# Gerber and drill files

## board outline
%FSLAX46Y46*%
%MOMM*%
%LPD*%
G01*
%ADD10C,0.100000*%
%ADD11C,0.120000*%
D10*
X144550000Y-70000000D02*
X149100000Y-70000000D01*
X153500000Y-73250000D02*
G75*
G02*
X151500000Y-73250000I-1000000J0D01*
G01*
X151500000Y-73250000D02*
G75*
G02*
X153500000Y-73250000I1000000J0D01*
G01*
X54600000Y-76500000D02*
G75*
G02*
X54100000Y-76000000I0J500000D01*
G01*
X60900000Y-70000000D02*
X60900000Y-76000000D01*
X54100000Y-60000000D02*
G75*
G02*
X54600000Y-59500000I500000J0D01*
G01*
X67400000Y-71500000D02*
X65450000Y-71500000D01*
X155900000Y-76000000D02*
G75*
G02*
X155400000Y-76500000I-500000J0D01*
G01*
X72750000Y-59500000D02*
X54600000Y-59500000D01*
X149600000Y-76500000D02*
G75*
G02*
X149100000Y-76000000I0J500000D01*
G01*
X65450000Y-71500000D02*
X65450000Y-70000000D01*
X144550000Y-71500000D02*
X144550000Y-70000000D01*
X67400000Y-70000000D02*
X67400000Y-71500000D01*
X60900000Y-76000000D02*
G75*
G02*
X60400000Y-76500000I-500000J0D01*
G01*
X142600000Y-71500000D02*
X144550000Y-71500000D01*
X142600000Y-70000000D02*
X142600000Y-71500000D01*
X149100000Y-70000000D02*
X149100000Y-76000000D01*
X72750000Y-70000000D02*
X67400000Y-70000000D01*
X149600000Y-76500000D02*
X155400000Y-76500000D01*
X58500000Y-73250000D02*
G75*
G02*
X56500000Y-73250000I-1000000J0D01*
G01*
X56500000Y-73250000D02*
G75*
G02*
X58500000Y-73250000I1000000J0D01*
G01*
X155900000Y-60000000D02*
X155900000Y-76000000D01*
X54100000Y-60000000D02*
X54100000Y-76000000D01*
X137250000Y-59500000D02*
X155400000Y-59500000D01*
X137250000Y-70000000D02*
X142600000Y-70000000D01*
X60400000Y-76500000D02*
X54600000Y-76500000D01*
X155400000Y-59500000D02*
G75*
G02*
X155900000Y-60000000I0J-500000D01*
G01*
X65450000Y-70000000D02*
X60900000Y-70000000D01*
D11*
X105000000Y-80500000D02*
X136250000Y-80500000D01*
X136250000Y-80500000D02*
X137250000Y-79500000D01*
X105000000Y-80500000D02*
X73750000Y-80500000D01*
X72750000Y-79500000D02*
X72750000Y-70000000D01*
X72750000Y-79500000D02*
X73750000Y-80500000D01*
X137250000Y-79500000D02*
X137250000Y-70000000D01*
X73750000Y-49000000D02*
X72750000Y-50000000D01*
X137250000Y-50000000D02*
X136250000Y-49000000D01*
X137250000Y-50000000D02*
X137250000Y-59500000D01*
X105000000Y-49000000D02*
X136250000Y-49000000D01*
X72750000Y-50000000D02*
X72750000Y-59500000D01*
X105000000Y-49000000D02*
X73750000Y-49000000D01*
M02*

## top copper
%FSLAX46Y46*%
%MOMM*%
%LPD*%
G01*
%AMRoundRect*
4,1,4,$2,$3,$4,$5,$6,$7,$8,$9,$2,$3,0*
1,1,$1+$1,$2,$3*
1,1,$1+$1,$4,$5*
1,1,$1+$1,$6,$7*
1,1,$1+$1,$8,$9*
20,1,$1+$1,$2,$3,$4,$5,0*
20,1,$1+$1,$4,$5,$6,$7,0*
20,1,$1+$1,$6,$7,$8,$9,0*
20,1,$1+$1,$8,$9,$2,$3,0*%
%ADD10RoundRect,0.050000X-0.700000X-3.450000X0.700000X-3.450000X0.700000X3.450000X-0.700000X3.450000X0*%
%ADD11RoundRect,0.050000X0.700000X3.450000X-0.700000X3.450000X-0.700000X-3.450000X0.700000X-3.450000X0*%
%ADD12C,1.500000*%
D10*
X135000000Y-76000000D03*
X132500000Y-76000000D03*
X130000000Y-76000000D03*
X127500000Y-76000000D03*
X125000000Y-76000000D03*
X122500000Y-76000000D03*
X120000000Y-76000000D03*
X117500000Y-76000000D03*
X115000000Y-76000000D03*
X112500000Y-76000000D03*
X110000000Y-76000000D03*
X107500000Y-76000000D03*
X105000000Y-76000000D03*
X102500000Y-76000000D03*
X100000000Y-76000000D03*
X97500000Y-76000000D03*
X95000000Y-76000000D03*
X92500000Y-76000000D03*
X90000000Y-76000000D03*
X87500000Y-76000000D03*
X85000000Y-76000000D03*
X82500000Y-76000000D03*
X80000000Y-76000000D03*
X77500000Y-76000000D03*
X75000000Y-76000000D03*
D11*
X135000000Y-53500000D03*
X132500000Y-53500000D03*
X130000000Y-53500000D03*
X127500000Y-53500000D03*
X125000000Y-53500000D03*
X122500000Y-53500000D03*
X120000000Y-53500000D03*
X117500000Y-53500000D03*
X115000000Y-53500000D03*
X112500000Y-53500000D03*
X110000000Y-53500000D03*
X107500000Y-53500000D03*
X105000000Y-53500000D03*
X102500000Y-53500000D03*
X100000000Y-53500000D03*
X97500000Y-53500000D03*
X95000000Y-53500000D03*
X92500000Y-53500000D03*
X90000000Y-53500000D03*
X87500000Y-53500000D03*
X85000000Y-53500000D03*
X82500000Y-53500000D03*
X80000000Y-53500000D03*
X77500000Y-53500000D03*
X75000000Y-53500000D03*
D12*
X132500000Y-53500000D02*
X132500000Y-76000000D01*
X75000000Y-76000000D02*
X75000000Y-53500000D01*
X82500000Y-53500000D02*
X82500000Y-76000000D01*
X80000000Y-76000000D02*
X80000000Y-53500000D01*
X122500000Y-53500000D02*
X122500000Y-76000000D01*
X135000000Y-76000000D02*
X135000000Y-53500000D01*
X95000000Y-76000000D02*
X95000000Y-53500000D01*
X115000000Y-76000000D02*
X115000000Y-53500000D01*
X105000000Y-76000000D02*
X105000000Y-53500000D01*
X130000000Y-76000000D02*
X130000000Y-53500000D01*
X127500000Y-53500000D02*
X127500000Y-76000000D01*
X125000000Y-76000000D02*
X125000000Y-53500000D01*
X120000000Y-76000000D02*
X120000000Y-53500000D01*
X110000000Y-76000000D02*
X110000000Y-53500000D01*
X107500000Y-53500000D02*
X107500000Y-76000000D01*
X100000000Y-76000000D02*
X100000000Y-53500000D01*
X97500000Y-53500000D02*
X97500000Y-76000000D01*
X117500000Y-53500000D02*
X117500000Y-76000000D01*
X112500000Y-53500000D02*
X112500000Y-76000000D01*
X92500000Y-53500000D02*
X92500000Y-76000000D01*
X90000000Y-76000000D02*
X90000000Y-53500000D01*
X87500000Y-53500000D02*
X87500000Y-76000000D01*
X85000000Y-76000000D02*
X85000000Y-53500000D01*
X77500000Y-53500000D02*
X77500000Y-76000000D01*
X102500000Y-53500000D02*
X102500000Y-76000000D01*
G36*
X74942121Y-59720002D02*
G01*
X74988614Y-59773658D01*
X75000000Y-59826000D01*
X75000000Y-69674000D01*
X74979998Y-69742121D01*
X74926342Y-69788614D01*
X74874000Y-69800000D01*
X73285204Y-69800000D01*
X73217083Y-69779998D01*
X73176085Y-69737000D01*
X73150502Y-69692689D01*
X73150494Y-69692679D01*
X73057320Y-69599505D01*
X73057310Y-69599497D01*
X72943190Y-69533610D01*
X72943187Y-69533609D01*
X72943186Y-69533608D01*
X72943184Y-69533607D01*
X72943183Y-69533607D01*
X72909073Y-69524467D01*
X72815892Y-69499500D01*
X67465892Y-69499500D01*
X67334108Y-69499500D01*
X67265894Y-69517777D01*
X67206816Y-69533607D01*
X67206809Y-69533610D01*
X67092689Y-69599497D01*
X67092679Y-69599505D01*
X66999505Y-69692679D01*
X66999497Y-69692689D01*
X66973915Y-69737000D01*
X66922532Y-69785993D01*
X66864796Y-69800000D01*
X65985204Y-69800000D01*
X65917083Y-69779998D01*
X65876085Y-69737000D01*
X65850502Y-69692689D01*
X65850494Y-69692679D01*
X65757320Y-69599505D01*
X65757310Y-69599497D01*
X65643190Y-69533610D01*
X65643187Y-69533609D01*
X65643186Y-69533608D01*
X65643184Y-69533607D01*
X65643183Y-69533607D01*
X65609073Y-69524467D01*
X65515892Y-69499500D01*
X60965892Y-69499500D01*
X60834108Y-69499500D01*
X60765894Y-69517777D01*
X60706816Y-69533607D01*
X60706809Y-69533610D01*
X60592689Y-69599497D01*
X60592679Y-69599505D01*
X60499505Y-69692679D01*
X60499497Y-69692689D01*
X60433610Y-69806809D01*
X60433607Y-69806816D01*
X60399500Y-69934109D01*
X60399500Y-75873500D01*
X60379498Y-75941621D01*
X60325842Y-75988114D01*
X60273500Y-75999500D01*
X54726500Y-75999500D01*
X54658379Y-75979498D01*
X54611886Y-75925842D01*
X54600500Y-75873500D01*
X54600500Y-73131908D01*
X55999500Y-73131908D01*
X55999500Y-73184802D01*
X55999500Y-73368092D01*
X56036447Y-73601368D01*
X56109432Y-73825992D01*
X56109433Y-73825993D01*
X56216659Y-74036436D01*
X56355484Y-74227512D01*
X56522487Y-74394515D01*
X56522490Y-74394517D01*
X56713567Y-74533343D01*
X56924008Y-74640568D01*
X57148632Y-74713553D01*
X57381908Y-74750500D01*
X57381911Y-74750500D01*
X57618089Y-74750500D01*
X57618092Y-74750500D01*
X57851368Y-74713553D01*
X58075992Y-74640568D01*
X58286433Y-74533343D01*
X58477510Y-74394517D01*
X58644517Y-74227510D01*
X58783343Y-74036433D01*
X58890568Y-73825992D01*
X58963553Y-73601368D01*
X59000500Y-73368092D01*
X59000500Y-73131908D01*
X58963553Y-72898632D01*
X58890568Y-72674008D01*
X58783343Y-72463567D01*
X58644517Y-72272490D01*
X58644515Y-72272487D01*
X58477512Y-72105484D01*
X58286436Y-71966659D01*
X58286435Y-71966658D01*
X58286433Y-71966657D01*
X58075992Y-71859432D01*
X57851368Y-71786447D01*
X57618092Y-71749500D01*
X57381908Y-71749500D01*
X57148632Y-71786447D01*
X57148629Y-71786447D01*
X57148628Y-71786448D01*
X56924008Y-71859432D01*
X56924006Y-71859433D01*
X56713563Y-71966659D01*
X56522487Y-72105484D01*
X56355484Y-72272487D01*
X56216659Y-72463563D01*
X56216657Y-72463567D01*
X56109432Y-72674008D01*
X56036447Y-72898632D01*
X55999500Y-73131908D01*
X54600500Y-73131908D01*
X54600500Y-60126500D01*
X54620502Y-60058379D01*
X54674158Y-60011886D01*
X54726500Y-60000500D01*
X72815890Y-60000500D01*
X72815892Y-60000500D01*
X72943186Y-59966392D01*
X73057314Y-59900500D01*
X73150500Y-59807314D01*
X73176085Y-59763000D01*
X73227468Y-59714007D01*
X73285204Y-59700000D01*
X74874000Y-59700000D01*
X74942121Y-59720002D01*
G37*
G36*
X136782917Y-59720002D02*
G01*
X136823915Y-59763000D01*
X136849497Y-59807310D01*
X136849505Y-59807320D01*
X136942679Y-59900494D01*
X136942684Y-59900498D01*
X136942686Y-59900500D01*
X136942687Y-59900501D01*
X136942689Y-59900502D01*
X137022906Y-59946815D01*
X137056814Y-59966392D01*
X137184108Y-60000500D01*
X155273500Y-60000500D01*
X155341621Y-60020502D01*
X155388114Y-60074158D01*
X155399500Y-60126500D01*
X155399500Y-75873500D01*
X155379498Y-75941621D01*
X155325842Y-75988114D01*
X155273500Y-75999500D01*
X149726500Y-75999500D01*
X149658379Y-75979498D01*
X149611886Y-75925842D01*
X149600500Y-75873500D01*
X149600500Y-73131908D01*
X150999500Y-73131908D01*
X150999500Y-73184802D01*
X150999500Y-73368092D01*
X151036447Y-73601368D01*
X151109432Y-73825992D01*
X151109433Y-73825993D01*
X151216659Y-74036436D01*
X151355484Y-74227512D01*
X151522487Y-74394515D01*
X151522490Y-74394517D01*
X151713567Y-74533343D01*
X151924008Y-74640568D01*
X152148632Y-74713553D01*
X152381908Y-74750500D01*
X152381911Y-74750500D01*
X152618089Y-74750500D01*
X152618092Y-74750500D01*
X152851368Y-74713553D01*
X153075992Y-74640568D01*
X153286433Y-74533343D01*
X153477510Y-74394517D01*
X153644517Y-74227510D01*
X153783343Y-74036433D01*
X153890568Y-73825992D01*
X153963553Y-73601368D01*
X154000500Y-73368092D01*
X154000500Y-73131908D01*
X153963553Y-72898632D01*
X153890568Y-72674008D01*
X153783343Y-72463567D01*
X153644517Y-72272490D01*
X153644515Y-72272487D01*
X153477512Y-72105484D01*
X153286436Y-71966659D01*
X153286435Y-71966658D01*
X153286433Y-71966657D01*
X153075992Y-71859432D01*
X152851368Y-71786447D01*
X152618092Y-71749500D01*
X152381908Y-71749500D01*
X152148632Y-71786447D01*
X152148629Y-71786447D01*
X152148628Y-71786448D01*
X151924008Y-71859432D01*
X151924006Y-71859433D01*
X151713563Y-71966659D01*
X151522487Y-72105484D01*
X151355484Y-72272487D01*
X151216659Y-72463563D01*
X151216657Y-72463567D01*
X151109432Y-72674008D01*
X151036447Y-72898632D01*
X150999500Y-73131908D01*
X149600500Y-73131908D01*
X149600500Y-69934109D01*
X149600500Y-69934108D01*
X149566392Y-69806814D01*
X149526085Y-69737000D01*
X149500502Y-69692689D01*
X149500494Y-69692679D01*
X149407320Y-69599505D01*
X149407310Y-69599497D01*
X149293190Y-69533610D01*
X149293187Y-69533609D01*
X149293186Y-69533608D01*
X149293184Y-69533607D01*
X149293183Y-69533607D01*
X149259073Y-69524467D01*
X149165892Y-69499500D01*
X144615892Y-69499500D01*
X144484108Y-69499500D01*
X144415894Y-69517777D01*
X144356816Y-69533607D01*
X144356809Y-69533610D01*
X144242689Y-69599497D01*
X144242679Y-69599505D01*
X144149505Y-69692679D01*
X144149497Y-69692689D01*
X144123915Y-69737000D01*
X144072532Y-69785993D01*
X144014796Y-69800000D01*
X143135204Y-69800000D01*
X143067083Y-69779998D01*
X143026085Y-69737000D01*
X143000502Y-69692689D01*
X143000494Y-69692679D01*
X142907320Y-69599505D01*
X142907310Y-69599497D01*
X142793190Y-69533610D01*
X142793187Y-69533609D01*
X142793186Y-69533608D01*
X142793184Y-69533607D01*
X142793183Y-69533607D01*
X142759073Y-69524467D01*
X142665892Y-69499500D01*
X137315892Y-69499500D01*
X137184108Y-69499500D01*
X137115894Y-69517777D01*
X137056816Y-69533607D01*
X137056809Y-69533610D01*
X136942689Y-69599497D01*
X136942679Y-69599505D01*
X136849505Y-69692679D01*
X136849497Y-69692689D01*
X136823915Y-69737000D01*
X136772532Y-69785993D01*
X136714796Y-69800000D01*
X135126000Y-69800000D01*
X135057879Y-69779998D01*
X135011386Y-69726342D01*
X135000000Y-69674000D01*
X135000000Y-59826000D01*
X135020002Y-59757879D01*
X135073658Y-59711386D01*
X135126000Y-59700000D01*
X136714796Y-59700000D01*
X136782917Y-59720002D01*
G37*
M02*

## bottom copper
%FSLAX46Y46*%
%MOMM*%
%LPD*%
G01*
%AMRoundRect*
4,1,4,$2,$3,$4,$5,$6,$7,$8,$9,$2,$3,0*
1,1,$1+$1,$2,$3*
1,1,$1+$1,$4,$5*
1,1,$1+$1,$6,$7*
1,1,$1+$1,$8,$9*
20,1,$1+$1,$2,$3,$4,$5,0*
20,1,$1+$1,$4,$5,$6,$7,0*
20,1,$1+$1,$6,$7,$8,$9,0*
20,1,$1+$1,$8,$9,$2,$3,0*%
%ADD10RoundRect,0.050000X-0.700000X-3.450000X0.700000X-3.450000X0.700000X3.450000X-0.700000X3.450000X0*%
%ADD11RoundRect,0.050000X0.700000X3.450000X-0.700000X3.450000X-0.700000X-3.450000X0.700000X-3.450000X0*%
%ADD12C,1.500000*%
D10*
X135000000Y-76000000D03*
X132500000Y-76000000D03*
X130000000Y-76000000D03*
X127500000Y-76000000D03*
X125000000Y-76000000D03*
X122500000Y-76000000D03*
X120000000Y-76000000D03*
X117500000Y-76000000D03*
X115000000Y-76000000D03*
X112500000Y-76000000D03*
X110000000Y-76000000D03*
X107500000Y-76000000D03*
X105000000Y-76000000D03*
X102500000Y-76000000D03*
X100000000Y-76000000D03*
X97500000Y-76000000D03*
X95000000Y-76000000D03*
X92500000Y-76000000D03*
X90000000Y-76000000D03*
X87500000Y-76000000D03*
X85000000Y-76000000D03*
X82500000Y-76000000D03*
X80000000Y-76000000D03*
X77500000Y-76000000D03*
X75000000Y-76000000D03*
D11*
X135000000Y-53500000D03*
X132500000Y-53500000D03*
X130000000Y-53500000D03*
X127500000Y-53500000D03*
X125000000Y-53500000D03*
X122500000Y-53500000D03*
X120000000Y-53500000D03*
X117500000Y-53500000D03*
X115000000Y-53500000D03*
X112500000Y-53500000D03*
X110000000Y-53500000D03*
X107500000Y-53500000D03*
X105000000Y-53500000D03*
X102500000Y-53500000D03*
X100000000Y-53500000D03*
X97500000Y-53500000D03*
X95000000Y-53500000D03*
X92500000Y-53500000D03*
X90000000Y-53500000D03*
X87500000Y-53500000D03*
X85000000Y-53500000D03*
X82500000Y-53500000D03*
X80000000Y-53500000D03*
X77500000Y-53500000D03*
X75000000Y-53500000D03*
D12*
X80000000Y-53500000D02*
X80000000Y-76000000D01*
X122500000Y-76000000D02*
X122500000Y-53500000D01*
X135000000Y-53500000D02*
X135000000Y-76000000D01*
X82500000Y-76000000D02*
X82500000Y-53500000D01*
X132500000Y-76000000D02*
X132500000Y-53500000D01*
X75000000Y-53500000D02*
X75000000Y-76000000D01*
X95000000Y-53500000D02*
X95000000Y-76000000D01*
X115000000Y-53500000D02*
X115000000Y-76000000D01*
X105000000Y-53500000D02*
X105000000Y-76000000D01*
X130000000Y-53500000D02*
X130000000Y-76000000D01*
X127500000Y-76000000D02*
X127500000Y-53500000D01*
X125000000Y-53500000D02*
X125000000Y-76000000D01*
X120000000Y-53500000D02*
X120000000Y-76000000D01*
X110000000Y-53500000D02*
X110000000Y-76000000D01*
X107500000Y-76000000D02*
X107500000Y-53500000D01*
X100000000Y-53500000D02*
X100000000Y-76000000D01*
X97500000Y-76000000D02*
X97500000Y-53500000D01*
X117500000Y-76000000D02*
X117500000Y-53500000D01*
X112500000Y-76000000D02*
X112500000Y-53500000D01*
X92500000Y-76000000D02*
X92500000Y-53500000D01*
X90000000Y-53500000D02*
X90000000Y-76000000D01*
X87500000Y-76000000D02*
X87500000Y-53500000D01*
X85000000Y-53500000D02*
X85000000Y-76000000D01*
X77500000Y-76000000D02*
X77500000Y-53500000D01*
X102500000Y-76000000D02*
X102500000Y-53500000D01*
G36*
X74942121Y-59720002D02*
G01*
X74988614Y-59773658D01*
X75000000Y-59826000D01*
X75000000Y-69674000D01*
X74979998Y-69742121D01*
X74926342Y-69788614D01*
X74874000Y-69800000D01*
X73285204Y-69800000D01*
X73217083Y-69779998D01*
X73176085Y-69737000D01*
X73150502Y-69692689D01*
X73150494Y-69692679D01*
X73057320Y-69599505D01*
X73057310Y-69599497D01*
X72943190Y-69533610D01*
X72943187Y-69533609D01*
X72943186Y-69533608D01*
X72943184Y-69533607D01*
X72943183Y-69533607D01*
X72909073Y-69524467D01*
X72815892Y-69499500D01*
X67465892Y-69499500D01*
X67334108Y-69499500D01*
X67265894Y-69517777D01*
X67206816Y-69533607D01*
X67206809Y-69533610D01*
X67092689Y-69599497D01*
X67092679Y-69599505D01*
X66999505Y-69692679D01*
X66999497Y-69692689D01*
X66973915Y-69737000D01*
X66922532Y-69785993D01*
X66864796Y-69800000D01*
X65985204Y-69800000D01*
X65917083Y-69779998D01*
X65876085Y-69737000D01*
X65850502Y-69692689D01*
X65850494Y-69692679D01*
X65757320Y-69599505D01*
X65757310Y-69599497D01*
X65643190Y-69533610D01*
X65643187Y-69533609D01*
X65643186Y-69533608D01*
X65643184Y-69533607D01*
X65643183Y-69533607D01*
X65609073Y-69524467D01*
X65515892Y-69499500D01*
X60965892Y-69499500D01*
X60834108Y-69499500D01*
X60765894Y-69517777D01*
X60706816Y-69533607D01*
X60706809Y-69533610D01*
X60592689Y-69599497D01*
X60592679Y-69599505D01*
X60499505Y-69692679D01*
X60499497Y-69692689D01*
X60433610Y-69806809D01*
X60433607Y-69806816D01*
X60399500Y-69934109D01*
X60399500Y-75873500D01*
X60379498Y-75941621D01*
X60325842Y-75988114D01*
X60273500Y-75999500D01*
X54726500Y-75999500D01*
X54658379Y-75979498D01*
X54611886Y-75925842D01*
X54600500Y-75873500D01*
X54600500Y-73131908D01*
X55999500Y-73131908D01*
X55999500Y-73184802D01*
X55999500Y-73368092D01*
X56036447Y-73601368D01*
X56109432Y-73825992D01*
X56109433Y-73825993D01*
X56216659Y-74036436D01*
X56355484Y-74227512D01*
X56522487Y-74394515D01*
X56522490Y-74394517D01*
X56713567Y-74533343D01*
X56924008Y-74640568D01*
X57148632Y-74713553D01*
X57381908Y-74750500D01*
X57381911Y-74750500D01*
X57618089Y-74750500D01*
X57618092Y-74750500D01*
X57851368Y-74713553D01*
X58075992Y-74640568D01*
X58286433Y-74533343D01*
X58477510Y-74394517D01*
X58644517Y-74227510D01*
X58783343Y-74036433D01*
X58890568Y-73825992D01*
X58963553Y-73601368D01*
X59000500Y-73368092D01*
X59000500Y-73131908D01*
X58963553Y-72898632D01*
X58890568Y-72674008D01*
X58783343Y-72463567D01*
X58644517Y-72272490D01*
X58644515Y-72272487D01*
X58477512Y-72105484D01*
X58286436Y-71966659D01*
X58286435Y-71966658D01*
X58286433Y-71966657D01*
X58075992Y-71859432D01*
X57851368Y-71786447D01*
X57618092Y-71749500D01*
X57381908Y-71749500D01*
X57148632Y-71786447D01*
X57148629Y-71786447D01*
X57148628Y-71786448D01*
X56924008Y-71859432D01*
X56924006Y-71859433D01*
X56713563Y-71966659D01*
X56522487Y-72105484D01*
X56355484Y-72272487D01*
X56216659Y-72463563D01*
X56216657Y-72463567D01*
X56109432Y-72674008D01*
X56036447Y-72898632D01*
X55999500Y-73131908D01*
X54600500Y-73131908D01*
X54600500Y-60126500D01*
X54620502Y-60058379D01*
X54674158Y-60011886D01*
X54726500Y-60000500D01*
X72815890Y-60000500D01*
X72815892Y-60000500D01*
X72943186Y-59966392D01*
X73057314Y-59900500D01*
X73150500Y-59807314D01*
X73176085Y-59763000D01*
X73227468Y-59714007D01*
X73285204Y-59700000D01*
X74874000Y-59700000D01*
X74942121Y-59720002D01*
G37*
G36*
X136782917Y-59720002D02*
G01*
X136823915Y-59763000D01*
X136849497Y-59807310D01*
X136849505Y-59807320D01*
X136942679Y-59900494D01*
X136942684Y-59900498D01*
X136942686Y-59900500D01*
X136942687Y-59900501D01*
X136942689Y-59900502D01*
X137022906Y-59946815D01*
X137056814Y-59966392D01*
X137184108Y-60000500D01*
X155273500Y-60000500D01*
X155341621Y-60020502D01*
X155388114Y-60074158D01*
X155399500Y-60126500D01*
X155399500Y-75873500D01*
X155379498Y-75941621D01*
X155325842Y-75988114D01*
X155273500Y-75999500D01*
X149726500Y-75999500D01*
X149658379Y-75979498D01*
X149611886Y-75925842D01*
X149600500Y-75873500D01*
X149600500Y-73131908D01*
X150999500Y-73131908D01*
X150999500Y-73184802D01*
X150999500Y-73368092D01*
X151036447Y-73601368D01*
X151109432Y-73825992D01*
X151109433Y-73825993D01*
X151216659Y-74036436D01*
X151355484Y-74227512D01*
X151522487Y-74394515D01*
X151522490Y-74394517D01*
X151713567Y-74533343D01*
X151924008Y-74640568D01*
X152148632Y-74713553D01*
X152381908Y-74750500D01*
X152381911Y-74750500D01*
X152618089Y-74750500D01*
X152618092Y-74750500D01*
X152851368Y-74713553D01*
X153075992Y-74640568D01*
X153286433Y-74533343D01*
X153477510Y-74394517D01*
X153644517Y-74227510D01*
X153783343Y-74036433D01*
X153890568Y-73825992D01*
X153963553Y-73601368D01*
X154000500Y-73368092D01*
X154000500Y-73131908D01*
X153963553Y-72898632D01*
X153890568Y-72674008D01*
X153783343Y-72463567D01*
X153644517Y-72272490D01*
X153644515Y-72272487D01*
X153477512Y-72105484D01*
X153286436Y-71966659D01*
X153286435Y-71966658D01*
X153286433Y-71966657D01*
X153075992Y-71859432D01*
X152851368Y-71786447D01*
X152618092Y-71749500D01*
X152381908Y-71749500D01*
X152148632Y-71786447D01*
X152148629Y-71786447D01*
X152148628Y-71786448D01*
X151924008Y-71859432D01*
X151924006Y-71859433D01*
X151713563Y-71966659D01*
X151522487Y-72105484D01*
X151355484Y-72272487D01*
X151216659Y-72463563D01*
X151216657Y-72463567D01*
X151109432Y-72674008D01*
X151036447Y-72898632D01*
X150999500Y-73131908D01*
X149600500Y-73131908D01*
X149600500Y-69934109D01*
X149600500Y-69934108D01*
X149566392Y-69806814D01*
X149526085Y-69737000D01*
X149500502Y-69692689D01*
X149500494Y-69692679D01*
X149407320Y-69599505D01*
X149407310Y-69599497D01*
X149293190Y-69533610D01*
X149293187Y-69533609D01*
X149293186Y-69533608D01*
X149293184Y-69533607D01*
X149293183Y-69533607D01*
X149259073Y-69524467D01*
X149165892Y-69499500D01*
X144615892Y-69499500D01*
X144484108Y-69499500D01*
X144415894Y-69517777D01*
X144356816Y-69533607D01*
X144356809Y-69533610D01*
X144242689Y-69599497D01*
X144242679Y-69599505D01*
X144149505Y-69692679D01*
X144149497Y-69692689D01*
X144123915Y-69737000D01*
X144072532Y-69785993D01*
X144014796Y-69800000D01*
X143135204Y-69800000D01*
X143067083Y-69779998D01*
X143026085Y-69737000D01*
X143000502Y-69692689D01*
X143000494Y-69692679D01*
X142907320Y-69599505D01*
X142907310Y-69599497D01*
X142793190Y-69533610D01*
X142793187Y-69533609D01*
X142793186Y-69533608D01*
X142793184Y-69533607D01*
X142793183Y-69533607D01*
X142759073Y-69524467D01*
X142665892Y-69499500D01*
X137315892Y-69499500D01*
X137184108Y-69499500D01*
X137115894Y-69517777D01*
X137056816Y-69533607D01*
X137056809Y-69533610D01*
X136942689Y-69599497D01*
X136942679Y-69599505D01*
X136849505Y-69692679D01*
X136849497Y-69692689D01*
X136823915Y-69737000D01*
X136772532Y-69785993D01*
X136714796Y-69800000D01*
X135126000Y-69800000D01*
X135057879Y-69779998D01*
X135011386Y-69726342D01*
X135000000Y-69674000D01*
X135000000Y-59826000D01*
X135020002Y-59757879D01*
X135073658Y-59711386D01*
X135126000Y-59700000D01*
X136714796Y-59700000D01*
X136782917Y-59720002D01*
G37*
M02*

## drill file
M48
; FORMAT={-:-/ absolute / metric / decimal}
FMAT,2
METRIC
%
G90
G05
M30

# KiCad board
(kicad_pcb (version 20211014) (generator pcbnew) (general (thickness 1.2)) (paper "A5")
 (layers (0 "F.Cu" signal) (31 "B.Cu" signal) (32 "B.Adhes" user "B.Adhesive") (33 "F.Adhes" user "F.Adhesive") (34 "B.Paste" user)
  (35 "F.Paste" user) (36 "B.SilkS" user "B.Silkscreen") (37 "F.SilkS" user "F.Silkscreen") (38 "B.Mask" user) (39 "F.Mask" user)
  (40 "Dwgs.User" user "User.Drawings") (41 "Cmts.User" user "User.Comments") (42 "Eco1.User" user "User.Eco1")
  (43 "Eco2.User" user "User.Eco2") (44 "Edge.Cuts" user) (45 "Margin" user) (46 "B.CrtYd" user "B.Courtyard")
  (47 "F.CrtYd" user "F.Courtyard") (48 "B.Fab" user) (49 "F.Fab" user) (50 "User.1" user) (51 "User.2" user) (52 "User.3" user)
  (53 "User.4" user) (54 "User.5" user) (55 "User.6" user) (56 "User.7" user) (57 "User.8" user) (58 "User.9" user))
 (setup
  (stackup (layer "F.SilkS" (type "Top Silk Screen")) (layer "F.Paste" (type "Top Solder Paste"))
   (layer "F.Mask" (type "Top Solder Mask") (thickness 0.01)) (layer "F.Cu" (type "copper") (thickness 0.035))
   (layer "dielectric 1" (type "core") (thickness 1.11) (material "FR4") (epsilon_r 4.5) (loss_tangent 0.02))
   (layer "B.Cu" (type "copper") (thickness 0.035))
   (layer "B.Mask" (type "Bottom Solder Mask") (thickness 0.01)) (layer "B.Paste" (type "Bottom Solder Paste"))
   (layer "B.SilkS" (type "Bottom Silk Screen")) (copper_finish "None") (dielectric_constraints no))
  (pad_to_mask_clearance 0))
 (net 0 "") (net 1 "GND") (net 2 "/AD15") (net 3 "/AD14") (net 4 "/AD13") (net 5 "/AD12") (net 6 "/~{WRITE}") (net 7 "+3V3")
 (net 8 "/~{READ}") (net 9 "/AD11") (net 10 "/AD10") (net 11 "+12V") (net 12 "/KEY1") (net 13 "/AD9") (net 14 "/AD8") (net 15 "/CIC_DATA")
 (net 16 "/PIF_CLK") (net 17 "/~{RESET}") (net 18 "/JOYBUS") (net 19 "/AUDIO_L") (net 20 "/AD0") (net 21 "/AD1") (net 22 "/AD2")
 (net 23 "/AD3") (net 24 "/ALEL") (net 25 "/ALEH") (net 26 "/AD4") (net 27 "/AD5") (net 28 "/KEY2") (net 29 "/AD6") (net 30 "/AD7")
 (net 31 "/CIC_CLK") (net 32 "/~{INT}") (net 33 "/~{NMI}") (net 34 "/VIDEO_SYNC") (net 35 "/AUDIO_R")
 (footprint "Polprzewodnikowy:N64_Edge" (layer "F.Cu") (at 105 70)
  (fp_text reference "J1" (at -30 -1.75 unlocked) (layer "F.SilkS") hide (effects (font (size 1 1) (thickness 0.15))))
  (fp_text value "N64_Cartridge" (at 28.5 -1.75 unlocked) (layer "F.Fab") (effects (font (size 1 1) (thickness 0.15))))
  (fp_line (start 0 10.5) (end 31.25 10.5) (layer "Edge.Cuts") (width 0.12))
  (fp_line (start 31.25 10.5) (end 32.25 9.5) (layer "Edge.Cuts") (width 0.12))
  (fp_line (start 0 10.5) (end -31.25 10.5) (layer "Edge.Cuts") (width 0.12))
  (fp_line (start -32.25 9.5) (end -32.25 0) (layer "Edge.Cuts") (width 0.12))
  (fp_line (start -32.25 9.5) (end -31.25 10.5) (layer "Edge.Cuts") (width 0.12))
  (fp_line (start 32.25 9.5) (end 32.25 0) (layer "Edge.Cuts") (width 0.12))
  (pad "1" connect roundrect (at 30 6) (size 1.5 7) (layers "B.Cu") (roundrect_rratio 0.03333333333) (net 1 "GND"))
  (pad "2" connect roundrect (at 27.5 6) (size 1.5 7) (layers "B.Cu") (roundrect_rratio 0.03333333333) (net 1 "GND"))
  (pad "3" connect roundrect (at 25 6) (size 1.5 7) (layers "B.Cu") (roundrect_rratio 0.03333333333) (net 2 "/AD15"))
  (pad "4" connect roundrect (at 22.5 6) (size 1.5 7) (layers "B.Cu") (roundrect_rratio 0.03333333333) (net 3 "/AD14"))
  (pad "5" connect roundrect (at 20 6) (size 1.5 7) (layers "B.Cu") (roundrect_rratio 0.03333333333) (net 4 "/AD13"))
  (pad "6" connect roundrect (at 17.5 6) (size 1.5 7) (layers "B.Cu") (roundrect_rratio 0.03333333333) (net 1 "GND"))
  (pad "7" connect roundrect (at 15 6) (size 1.5 7) (layers "B.Cu") (roundrect_rratio 0.03333333333) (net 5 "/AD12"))
  (pad "8" connect roundrect (at 12.5 6) (size 1.5 7) (layers "B.Cu") (roundrect_rratio 0.03333333333) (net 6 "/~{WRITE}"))
  (pad "9" connect roundrect (at 10 6) (size 1.5 7) (layers "B.Cu") (roundrect_rratio 0.03333333333) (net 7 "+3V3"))
  (pad "10" connect roundrect (at 7.5 6) (size 1.5 7) (layers "B.Cu") (roundrect_rratio 0.03333333333) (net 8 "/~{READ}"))
  (pad "11" connect roundrect (at 5 6) (size 1.5 7) (layers "B.Cu") (roundrect_rratio 0.03333333333) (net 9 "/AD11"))
  (pad "12" connect roundrect (at 2.5 6) (size 1.5 7) (layers "B.Cu") (roundrect_rratio 0.03333333333) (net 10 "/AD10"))
  (pad "13" connect roundrect (at 0 6) (size 1.5 7) (layers "B.Cu") (roundrect_rratio 0.03333333333) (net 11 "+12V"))
  (pad "14" connect roundrect (at -2.5 6) (size 1.5 7) (layers "B.Cu") (roundrect_rratio 0.03333333333) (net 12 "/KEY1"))
  (pad "15" connect roundrect (at -5 6) (size 1.5 7) (layers "B.Cu") (roundrect_rratio 0.03333333333) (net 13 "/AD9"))
  (pad "16" connect roundrect (at -7.5 6) (size 1.5 7) (layers "B.Cu") (roundrect_rratio 0.03333333333) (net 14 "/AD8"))
  (pad "17" connect roundrect (at -10 6) (size 1.5 7) (layers "B.Cu") (roundrect_rratio 0.03333333333) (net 7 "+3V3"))
  (pad "18" connect roundrect (at -12.5 6) (size 1.5 7) (layers "B.Cu") (roundrect_rratio 0.03333333333) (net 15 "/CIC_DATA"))
  (pad "19" connect roundrect (at -15 6) (size 1.5 7) (layers "B.Cu") (roundrect_rratio 0.03333333333) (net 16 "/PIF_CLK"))
  (pad "20" connect roundrect (at -17.5 6) (size 1.5 7) (layers "B.Cu") (roundrect_rratio 0.03333333333) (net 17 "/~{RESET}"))
  (pad "21" connect roundrect (at -20 6) (size 1.5 7) (layers "B.Cu") (roundrect_rratio 0.03333333333) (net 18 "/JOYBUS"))
  (pad "22" connect roundrect (at -22.5 6) (size 1.5 7) (layers "B.Cu") (roundrect_rratio 0.03333333333) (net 1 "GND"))
  (pad "23" connect roundrect (at -25 6) (size 1.5 7) (layers "B.Cu") (roundrect_rratio 0.03333333333) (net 1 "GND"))
  (pad "24" connect roundrect (at -27.5 6) (size 1.5 7) (layers "B.Cu") (roundrect_rratio 0.03333333333) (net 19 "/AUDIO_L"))
  (pad "25" connect roundrect (at -30 6) (size 1.5 7) (layers "B.Cu") (roundrect_rratio 0.03333333333) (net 1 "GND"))
  (pad "26" connect roundrect (at 30 6) (size 1.5 7) (layers "F.Cu") (roundrect_rratio 0.03333333333) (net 1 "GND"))
  (pad "27" connect roundrect (at 27.5 6) (size 1.5 7) (layers "F.Cu") (roundrect_rratio 0.03333333333) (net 1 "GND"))
  (pad "28" connect roundrect (at 25 6) (size 1.5 7) (layers "F.Cu") (roundrect_rratio 0.03333333333) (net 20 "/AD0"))
  (pad "29" connect roundrect (at 22.5 6) (size 1.5 7) (layers "F.Cu") (roundrect_rratio 0.03333333333) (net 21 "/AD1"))
  (pad "30" connect roundrect (at 20 6) (size 1.5 7) (layers "F.Cu") (roundrect_rratio 0.03333333333) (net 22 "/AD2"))
  (pad "31" connect roundrect (at 17.5 6) (size 1.5 7) (layers "F.Cu") (roundrect_rratio 0.03333333333) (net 1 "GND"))
  (pad "32" connect roundrect (at 15 6) (size 1.5 7) (layers "F.Cu") (roundrect_rratio 0.03333333333) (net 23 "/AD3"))
  (pad "33" connect roundrect (at 12.5 6) (size 1.5 7) (layers "F.Cu") (roundrect_rratio 0.03333333333) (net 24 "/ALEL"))
  (pad "34" connect roundrect (at 10 6) (size 1.5 7) (layers "F.Cu") (roundrect_rratio 0.03333333333) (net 7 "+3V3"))
  (pad "35" connect roundrect (at 7.5 6) (size 1.5 7) (layers "F.Cu") (roundrect_rratio 0.03333333333) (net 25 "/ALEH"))
  (pad "36" connect roundrect (at 5 6) (size 1.5 7) (layers "F.Cu") (roundrect_rratio 0.03333333333) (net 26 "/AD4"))
  (pad "37" connect roundrect (at 2.5 6) (size 1.5 7) (layers "F.Cu") (roundrect_rratio 0.03333333333) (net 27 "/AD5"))
  (pad "38" connect roundrect (at 0 6) (size 1.5 7) (layers "F.Cu") (roundrect_rratio 0.03333333333) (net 11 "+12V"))
  (pad "39" connect roundrect (at -2.5 6) (size 1.5 7) (layers "F.Cu") (roundrect_rratio 0.03333333333) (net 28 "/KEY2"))
  (pad "40" connect roundrect (at -5 6) (size 1.5 7) (layers "F.Cu") (roundrect_rratio 0.03333333333) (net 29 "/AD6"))
  (pad "41" connect roundrect (at -7.5 6) (size 1.5 7) (layers "F.Cu") (roundrect_rratio 0.03333333333) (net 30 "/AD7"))
  (pad "42" connect roundrect (at -10 6) (size 1.5 7) (layers "F.Cu") (roundrect_rratio 0.03333333333) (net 7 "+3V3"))
  (pad "43" connect roundrect (at -12.5 6) (size 1.5 7) (layers "F.Cu") (roundrect_rratio 0.03333333333) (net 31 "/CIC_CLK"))
  (pad "44" connect roundrect (at -15 6) (size 1.5 7) (layers "F.Cu") (roundrect_rratio 0.03333333333) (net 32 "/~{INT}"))
  (pad "45" connect roundrect (at -17.5 6) (size 1.5 7) (layers "F.Cu") (roundrect_rratio 0.03333333333) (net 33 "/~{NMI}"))
  (pad "46" connect roundrect (at -20 6) (size 1.5 7) (layers "F.Cu") (roundrect_rratio 0.03333333333) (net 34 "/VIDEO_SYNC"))
  (pad "47" connect roundrect (at -22.5 6) (size 1.5 7) (layers "F.Cu") (roundrect_rratio 0.03333333333) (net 1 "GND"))
  (pad "48" connect roundrect (at -25 6) (size 1.5 7) (layers "F.Cu") (roundrect_rratio 0.03333333333) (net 1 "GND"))
  (pad "49" connect roundrect (at -27.5 6) (size 1.5 7) (layers "F.Cu") (roundrect_rratio 0.03333333333) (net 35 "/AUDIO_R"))
  (pad "50" connect roundrect (at -30 6) (size 1.5 7) (layers "F.Cu") (roundrect_rratio 0.03333333333) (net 1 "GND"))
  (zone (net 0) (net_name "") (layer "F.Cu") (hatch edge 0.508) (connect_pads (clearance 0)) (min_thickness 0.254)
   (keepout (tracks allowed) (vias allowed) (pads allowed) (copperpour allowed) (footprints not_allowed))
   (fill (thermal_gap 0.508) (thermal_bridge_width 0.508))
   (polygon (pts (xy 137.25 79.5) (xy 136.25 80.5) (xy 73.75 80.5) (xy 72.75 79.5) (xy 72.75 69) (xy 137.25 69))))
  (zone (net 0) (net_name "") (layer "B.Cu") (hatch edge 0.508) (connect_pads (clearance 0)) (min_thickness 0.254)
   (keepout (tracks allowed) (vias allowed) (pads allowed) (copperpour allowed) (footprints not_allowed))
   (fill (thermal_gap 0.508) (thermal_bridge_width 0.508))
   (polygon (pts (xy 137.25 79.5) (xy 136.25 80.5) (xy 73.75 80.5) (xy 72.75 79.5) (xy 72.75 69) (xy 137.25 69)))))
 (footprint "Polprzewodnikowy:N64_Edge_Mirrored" (layer "F.Cu") (at 105 59.5 180)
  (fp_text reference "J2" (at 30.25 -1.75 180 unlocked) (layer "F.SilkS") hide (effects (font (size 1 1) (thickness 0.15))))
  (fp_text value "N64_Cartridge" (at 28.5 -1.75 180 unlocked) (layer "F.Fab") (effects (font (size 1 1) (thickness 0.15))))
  (fp_line (start 31.25 10.5) (end 32.25 9.5) (layer "Edge.Cuts") (width 0.12))
  (fp_line (start -32.25 9.5) (end -31.25 10.5) (layer "Edge.Cuts") (width 0.12))
  (fp_line (start -32.25 9.5) (end -32.25 0) (layer "Edge.Cuts") (width 0.12))
  (fp_line (start 0 10.5) (end -31.25 10.5) (layer "Edge.Cuts") (width 0.12))
  (fp_line (start 32.25 9.5) (end 32.25 0) (layer "Edge.Cuts") (width 0.12))
  (fp_line (start 0 10.5) (end 31.25 10.5) (layer "Edge.Cuts") (width 0.12))
  (pad "1" connect roundrect (at -30 6 180) (size 1.5 7) (layers "B.Cu") (roundrect_rratio 0.03333333333) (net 1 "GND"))
  (pad "2" connect roundrect (at -27.5 6 180) (size 1.5 7) (layers "B.Cu") (roundrect_rratio 0.03333333333) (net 1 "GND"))
  (pad "3" connect roundrect (at -25 6 180) (size 1.5 7) (layers "B.Cu") (roundrect_rratio 0.03333333333) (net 2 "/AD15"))
  (pad "4" connect roundrect (at -22.5 6 180) (size 1.5 7) (layers "B.Cu") (roundrect_rratio 0.03333333333) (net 3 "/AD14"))
  (pad "5" connect roundrect (at -20 6 180) (size 1.5 7) (layers "B.Cu") (roundrect_rratio 0.03333333333) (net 4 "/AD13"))
  (pad "6" connect roundrect (at -17.5 6 180) (size 1.5 7) (layers "B.Cu") (roundrect_rratio 0.03333333333) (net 1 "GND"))
  (pad "7" connect roundrect (at -15 6 180) (size 1.5 7) (layers "B.Cu") (roundrect_rratio 0.03333333333) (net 5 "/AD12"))
  (pad "8" connect roundrect (at -12.5 6 180) (size 1.5 7) (layers "B.Cu") (roundrect_rratio 0.03333333333) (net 6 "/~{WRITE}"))
  (pad "9" connect roundrect (at -10 6 180) (size 1.5 7) (layers "B.Cu") (roundrect_rratio 0.03333333333) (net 7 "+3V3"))
  (pad "10" connect roundrect (at -7.5 6 180) (size 1.5 7) (layers "B.Cu") (roundrect_rratio 0.03333333333) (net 8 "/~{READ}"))
  (pad "11" connect roundrect (at -5 6 180) (size 1.5 7) (layers "B.Cu") (roundrect_rratio 0.03333333333) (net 9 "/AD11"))
  (pad "12" connect roundrect (at -2.5 6 180) (size 1.5 7) (layers "B.Cu") (roundrect_rratio 0.03333333333) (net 10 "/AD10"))
  (pad "13" connect roundrect (at 0 6 180) (size 1.5 7) (layers "B.Cu") (roundrect_rratio 0.03333333333) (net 11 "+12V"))
  (pad "14" connect roundrect (at 2.5 6 180) (size 1.5 7) (layers "B.Cu") (roundrect_rratio 0.03333333333) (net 12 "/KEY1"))
  (pad "15" connect roundrect (at 5 6 180) (size 1.5 7) (layers "B.Cu") (roundrect_rratio 0.03333333333) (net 13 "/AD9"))
  (pad "16" connect roundrect (at 7.5 6 180) (size 1.5 7) (layers "B.Cu") (roundrect_rratio 0.03333333333) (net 14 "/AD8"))
  (pad "17" connect roundrect (at 10 6 180) (size 1.5 7) (layers "B.Cu") (roundrect_rratio 0.03333333333) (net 7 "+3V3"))
  (pad "18" connect roundrect (at 12.5 6 180) (size 1.5 7) (layers "B.Cu") (roundrect_rratio 0.03333333333) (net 15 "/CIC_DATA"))
  (pad "19" connect roundrect (at 15 6 180) (size 1.5 7) (layers "B.Cu") (roundrect_rratio 0.03333333333) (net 16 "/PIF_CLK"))
  (pad "20" connect roundrect (at 17.5 6 180) (size 1.5 7) (layers "B.Cu") (roundrect_rratio 0.03333333333) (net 17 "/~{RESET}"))
  (pad "21" connect roundrect (at 20 6 180) (size 1.5 7) (layers "B.Cu") (roundrect_rratio 0.03333333333) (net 18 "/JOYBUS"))
  (pad "22" connect roundrect (at 22.5 6 180) (size 1.5 7) (layers "B.Cu") (roundrect_rratio 0.03333333333) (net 1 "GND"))
  (pad "23" connect roundrect (at 25 6 180) (size 1.5 7) (layers "B.Cu") (roundrect_rratio 0.03333333333) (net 1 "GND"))
  (pad "24" connect roundrect (at 27.5 6 180) (size 1.5 7) (layers "B.Cu") (roundrect_rratio 0.03333333333) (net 19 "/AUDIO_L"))
  (pad "25" connect roundrect (at 30 6 180) (size 1.5 7) (layers "B.Cu") (roundrect_rratio 0.03333333333) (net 1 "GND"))
  (pad "26" connect roundrect (at -30 6 180) (size 1.5 7) (layers "F.Cu") (roundrect_rratio 0.03333333333) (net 1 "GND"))
  (pad "27" connect roundrect (at -27.5 6 180) (size 1.5 7) (layers "F.Cu") (roundrect_rratio 0.03333333333) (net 1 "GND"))
  (pad "28" connect roundrect (at -25 6 180) (size 1.5 7) (layers "F.Cu") (roundrect_rratio 0.03333333333) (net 20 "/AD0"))
  (pad "29" connect roundrect (at -22.5 6 180) (size 1.5 7) (layers "F.Cu") (roundrect_rratio 0.03333333333) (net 21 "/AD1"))
  (pad "30" connect roundrect (at -20 6 180) (size 1.5 7) (layers "F.Cu") (roundrect_rratio 0.03333333333) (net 22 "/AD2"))
  (pad "31" connect roundrect (at -17.5 6 180) (size 1.5 7) (layers "F.Cu") (roundrect_rratio 0.03333333333) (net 1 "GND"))
  (pad "32" connect roundrect (at -15 6 180) (size 1.5 7) (layers "F.Cu") (roundrect_rratio 0.03333333333) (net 23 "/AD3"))
  (pad "33" connect roundrect (at -12.5 6 180) (size 1.5 7) (layers "F.Cu") (roundrect_rratio 0.03333333333) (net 24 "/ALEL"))
  (pad "34" connect roundrect (at -10 6 180) (size 1.5 7) (layers "F.Cu") (roundrect_rratio 0.03333333333) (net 7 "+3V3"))
  (pad "35" connect roundrect (at -7.5 6 180) (size 1.5 7) (layers "F.Cu") (roundrect_rratio 0.03333333333) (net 25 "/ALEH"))
  (pad "36" connect roundrect (at -5 6 180) (size 1.5 7) (layers "F.Cu") (roundrect_rratio 0.03333333333) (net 26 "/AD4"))
  (pad "37" connect roundrect (at -2.5 6 180) (size 1.5 7) (layers "F.Cu") (roundrect_rratio 0.03333333333) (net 27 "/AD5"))
  (pad "38" connect roundrect (at 0 6 180) (size 1.5 7) (layers "F.Cu") (roundrect_rratio 0.03333333333) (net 11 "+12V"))
  (pad "39" connect roundrect (at 2.5 6 180) (size 1.5 7) (layers "F.Cu") (roundrect_rratio 0.03333333333) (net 28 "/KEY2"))
  (pad "40" connect roundrect (at 5 6 180) (size 1.5 7) (layers "F.Cu") (roundrect_rratio 0.03333333333) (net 29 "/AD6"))
  (pad "41" connect roundrect (at 7.5 6 180) (size 1.5 7) (layers "F.Cu") (roundrect_rratio 0.03333333333) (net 30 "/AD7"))
  (pad "42" connect roundrect (at 10 6 180) (size 1.5 7) (layers "F.Cu") (roundrect_rratio 0.03333333333) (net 7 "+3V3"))
  (pad "43" connect roundrect (at 12.5 6 180) (size 1.5 7) (layers "F.Cu") (roundrect_rratio 0.03333333333) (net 31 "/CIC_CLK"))
  (pad "44" connect roundrect (at 15 6 180) (size 1.5 7) (layers "F.Cu") (roundrect_rratio 0.03333333333) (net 32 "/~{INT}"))
  (pad "45" connect roundrect (at 17.5 6 180) (size 1.5 7) (layers "F.Cu") (roundrect_rratio 0.03333333333) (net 33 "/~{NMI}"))
  (pad "46" connect roundrect (at 20 6 180) (size 1.5 7) (layers "F.Cu") (roundrect_rratio 0.03333333333) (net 34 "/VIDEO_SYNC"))
  (pad "47" connect roundrect (at 22.5 6 180) (size 1.5 7) (layers "F.Cu") (roundrect_rratio 0.03333333333) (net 1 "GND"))
  (pad "48" connect roundrect (at 25 6 180) (size 1.5 7) (layers "F.Cu") (roundrect_rratio 0.03333333333) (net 1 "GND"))
  (pad "49" connect roundrect (at 27.5 6 180) (size 1.5 7) (layers "F.Cu") (roundrect_rratio 0.03333333333) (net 35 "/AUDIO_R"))
  (pad "50" connect roundrect (at 30 6 180) (size 1.5 7) (layers "F.Cu") (roundrect_rratio 0.03333333333) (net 1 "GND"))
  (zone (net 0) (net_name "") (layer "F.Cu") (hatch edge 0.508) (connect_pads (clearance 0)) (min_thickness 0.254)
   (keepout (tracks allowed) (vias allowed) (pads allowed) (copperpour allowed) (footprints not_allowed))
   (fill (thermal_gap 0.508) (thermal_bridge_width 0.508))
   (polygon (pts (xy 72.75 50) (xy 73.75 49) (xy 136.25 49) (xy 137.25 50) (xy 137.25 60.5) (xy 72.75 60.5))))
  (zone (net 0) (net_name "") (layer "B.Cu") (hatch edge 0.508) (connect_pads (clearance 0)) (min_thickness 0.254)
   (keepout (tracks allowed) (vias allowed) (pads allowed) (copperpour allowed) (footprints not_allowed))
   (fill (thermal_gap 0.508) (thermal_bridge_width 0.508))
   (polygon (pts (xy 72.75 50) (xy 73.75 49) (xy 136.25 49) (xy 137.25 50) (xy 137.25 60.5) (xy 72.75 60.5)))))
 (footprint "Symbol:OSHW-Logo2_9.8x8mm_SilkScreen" (layer "B.Cu") (at 66.5 64.75 180)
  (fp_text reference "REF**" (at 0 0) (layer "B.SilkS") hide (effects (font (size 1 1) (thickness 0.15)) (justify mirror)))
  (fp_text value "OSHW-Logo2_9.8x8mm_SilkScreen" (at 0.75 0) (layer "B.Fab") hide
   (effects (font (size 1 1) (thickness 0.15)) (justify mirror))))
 (gr_line (start 144.55 70) (end 149.1 70) (layer "Edge.Cuts") (width 0.1))
 (gr_circle (center 152.5 73.25) (end 153.5 73.25) (layer "Edge.Cuts") (width 0.1) (fill none))
 (gr_arc (start 54.6 76.5) (mid 54.246447 76.353553) (end 54.1 76) (layer "Edge.Cuts") (width 0.1))
 (gr_line (start 60.9 70) (end 60.9 76) (layer "Edge.Cuts") (width 0.1))
 (gr_arc (start 54.1 60) (mid 54.246447 59.646447) (end 54.6 59.5) (layer "Edge.Cuts") (width 0.1))
 (gr_line (start 67.4 71.5) (end 65.45 71.5) (layer "Edge.Cuts") (width 0.1))
 (gr_arc (start 155.9 76) (mid 155.753553 76.353553) (end 155.4 76.5) (layer "Edge.Cuts") (width 0.1))
 (gr_line (start 72.75 59.5) (end 54.6 59.5) (layer "Edge.Cuts") (width 0.1))
 (gr_arc (start 149.6 76.5) (mid 149.246447 76.353553) (end 149.1 76) (layer "Edge.Cuts") (width 0.1))
 (gr_line (start 65.45 71.5) (end 65.45 70) (layer "Edge.Cuts") (width 0.1))
 (gr_line (start 144.55 71.5) (end 144.55 70) (layer "Edge.Cuts") (width 0.1))
 (gr_line (start 67.4 70) (end 67.4 71.5) (layer "Edge.Cuts") (width 0.1))
 (gr_arc (start 60.9 76) (mid 60.753553 76.353553) (end 60.4 76.5) (layer "Edge.Cuts") (width 0.1))
 (gr_line (start 142.6 71.5) (end 144.55 71.5) (layer "Edge.Cuts") (width 0.1))
 (gr_line (start 142.6 70) (end 142.6 71.5) (layer "Edge.Cuts") (width 0.1))
 (gr_line (start 149.1 70) (end 149.1 76) (layer "Edge.Cuts") (width 0.1))
 (gr_line (start 72.75 70) (end 67.4 70) (layer "Edge.Cuts") (width 0.1))
 (gr_line (start 149.6 76.5) (end 155.4 76.5) (layer "Edge.Cuts") (width 0.1))
 (gr_circle (center 57.5 73.25) (end 58.5 73.25) (layer "Edge.Cuts") (width 0.1) (fill none))
 (gr_line (start 155.9 60) (end 155.9 76) (layer "Edge.Cuts") (width 0.1))
 (gr_line (start 54.1 60) (end 54.1 76) (layer "Edge.Cuts") (width 0.1))
 (gr_line (start 137.25 59.5) (end 155.4 59.5) (layer "Edge.Cuts") (width 0.1))
 (gr_line (start 137.25 70) (end 142.6 70) (layer "Edge.Cuts") (width 0.1))
 (gr_line (start 60.4 76.5) (end 54.6 76.5) (layer "Edge.Cuts") (width 0.1))
 (gr_arc (start 155.4 59.5) (mid 155.753553 59.646447) (end 155.9 60) (layer "Edge.Cuts") (width 0.1))
 (gr_line (start 65.45 70) (end 60.9 70) (layer "Edge.Cuts") (width 0.1))
 (segment (start 132.5 53.5) (end 132.5 76) (width 1.5) (layer "F.Cu") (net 1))
 (segment (start 75 76) (end 75 53.5) (width 1.5) (layer "F.Cu") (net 1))
 (segment (start 82.5 53.5) (end 82.5 76) (width 1.5) (layer "F.Cu") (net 1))
 (segment (start 80 76) (end 80 53.5) (width 1.5) (layer "F.Cu") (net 1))
 (segment (start 122.5 53.5) (end 122.5 76) (width 1.5) (layer "F.Cu") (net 1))
 (segment (start 135 76) (end 135 53.5) (width 1.5) (layer "F.Cu") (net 1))
 (segment (start 80 53.5) (end 80 76) (width 1.5) (layer "B.Cu") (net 1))
 (segment (start 122.5 76) (end 122.5 53.5) (width 1.5) (layer "B.Cu") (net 1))
 (segment (start 135 53.5) (end 135 76) (width 1.5) (layer "B.Cu") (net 1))
 (segment (start 82.5 76) (end 82.5 53.5) (width 1.5) (layer "B.Cu") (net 1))
 (segment (start 132.5 76) (end 132.5 53.5) (width 1.5) (layer "B.Cu") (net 1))
 (segment (start 75 53.5) (end 75 76) (width 1.5) (layer "B.Cu") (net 1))
 (segment (start 95 76) (end 95 53.5) (width 1.5) (layer "F.Cu") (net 7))
 (segment (start 115 76) (end 115 53.5) (width 1.5) (layer "F.Cu") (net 7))
 (segment (start 95 53.5) (end 95 76) (width 1.5) (layer "B.Cu") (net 7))
 (segment (start 115 53.5) (end 115 76) (width 1.5) (layer "B.Cu") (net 7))
 (segment (start 105 76) (end 105 53.5) (width 1.5) (layer "F.Cu") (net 11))
 (segment (start 105 53.5) (end 105 76) (width 1.5) (layer "B.Cu") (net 11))
 (segment (start 130 76) (end 130 53.5) (width 1.5) (layer "F.Cu") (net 20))
 (segment (start 127.5 53.5) (end 127.5 76) (width 1.5) (layer "F.Cu") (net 21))
 (segment (start 130 53.5) (end 130 76) (width 1.5) (layer "B.Cu") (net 2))
 (segment (start 127.5 76) (end 127.5 53.5) (width 1.5) (layer "B.Cu") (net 3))
 (segment (start 125 53.5) (end 125 76) (width 1.5) (layer "B.Cu") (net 4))
 (segment (start 120 53.5) (end 120 76) (width 1.5) (layer "B.Cu") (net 5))
 (segment (start 110 53.5) (end 110 76) (width 1.5) (layer "B.Cu") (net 9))
 (segment (start 107.5 76) (end 107.5 53.5) (width 1.5) (layer "B.Cu") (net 10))
 (segment (start 100 53.5) (end 100 76) (width 1.5) (layer "B.Cu") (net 13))
 (segment (start 97.5 76) (end 97.5 53.5) (width 1.5) (layer "B.Cu") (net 14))
 (segment (start 125 76) (end 125 53.5) (width 1.5) (layer "F.Cu") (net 22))
 (segment (start 120 76) (end 120 53.5) (width 1.5) (layer "F.Cu") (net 23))
 (segment (start 110 76) (end 110 53.5) (width 1.5) (layer "F.Cu") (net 26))
 (segment (start 107.5 53.5) (end 107.5 76) (width 1.5) (layer "F.Cu") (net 27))
 (segment (start 100 76) (end 100 53.5) (width 1.5) (layer "F.Cu") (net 29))
 (segment (start 97.5 53.5) (end 97.5 76) (width 1.5) (layer "F.Cu") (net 30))
 (segment (start 117.5 76) (end 117.5 53.5) (width 1.5) (layer "B.Cu") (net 6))
 (segment (start 112.5 76) (end 112.5 53.5) (width 1.5) (layer "B.Cu") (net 8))
 (segment (start 92.5 76) (end 92.5 53.5) (width 1.5) (layer "B.Cu") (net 15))
 (segment (start 90 53.5) (end 90 76) (width 1.5) (layer "B.Cu") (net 16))
 (segment (start 87.5 76) (end 87.5 53.5) (width 1.5) (layer "B.Cu") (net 17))
 (segment (start 85 53.5) (end 85 76) (width 1.5) (layer "B.Cu") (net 18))
 (segment (start 77.5 76) (end 77.5 53.5) (width 1.5) (layer "B.Cu") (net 19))
 (segment (start 117.5 53.5) (end 117.5 76) (width 1.5) (layer "F.Cu") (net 24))
 (segment (start 112.5 53.5) (end 112.5 76) (width 1.5) (layer "F.Cu") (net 25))
 (segment (start 92.5 53.5) (end 92.5 76) (width 1.5) (layer "F.Cu") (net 31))
 (segment (start 90 76) (end 90 53.5) (width 1.5) (layer "F.Cu") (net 32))
 (segment (start 87.5 53.5) (end 87.5 76) (width 1.5) (layer "F.Cu") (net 33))
 (segment (start 85 76) (end 85 53.5) (width 1.5) (layer "F.Cu") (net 34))
 (segment (start 77.5 53.5) (end 77.5 76) (width 1.5) (layer "F.Cu") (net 35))
 (segment (start 102.5 76) (end 102.5 53.5) (width 1.5) (layer "B.Cu") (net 12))
 (segment (start 102.5 53.5) (end 102.5 76) (width 1.5) (layer "F.Cu") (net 28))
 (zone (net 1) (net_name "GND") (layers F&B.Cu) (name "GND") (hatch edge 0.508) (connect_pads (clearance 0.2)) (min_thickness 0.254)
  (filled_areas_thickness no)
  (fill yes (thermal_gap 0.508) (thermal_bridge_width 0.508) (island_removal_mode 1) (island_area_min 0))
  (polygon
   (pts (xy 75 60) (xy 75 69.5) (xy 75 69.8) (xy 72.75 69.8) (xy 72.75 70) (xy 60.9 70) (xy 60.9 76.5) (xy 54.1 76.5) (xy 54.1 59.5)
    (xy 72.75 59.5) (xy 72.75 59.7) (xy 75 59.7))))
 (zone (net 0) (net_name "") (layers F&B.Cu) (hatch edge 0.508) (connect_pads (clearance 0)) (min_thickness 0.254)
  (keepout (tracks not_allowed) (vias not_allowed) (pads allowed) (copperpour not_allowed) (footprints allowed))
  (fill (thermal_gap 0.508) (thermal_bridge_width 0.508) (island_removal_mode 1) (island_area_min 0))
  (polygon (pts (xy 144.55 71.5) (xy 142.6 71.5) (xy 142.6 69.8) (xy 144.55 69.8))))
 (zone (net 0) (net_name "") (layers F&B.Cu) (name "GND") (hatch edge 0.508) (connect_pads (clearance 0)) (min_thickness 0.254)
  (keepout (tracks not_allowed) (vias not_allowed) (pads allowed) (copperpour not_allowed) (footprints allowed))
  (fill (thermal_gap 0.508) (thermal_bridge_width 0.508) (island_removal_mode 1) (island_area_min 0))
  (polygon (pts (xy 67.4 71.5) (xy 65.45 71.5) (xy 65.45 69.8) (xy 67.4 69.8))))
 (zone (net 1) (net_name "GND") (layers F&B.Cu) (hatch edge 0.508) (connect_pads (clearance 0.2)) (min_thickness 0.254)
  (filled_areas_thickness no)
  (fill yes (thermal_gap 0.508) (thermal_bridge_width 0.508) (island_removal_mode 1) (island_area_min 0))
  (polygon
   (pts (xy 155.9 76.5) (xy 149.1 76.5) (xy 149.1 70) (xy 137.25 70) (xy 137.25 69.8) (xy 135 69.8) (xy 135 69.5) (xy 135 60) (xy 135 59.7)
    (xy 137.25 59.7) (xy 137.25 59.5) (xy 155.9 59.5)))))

